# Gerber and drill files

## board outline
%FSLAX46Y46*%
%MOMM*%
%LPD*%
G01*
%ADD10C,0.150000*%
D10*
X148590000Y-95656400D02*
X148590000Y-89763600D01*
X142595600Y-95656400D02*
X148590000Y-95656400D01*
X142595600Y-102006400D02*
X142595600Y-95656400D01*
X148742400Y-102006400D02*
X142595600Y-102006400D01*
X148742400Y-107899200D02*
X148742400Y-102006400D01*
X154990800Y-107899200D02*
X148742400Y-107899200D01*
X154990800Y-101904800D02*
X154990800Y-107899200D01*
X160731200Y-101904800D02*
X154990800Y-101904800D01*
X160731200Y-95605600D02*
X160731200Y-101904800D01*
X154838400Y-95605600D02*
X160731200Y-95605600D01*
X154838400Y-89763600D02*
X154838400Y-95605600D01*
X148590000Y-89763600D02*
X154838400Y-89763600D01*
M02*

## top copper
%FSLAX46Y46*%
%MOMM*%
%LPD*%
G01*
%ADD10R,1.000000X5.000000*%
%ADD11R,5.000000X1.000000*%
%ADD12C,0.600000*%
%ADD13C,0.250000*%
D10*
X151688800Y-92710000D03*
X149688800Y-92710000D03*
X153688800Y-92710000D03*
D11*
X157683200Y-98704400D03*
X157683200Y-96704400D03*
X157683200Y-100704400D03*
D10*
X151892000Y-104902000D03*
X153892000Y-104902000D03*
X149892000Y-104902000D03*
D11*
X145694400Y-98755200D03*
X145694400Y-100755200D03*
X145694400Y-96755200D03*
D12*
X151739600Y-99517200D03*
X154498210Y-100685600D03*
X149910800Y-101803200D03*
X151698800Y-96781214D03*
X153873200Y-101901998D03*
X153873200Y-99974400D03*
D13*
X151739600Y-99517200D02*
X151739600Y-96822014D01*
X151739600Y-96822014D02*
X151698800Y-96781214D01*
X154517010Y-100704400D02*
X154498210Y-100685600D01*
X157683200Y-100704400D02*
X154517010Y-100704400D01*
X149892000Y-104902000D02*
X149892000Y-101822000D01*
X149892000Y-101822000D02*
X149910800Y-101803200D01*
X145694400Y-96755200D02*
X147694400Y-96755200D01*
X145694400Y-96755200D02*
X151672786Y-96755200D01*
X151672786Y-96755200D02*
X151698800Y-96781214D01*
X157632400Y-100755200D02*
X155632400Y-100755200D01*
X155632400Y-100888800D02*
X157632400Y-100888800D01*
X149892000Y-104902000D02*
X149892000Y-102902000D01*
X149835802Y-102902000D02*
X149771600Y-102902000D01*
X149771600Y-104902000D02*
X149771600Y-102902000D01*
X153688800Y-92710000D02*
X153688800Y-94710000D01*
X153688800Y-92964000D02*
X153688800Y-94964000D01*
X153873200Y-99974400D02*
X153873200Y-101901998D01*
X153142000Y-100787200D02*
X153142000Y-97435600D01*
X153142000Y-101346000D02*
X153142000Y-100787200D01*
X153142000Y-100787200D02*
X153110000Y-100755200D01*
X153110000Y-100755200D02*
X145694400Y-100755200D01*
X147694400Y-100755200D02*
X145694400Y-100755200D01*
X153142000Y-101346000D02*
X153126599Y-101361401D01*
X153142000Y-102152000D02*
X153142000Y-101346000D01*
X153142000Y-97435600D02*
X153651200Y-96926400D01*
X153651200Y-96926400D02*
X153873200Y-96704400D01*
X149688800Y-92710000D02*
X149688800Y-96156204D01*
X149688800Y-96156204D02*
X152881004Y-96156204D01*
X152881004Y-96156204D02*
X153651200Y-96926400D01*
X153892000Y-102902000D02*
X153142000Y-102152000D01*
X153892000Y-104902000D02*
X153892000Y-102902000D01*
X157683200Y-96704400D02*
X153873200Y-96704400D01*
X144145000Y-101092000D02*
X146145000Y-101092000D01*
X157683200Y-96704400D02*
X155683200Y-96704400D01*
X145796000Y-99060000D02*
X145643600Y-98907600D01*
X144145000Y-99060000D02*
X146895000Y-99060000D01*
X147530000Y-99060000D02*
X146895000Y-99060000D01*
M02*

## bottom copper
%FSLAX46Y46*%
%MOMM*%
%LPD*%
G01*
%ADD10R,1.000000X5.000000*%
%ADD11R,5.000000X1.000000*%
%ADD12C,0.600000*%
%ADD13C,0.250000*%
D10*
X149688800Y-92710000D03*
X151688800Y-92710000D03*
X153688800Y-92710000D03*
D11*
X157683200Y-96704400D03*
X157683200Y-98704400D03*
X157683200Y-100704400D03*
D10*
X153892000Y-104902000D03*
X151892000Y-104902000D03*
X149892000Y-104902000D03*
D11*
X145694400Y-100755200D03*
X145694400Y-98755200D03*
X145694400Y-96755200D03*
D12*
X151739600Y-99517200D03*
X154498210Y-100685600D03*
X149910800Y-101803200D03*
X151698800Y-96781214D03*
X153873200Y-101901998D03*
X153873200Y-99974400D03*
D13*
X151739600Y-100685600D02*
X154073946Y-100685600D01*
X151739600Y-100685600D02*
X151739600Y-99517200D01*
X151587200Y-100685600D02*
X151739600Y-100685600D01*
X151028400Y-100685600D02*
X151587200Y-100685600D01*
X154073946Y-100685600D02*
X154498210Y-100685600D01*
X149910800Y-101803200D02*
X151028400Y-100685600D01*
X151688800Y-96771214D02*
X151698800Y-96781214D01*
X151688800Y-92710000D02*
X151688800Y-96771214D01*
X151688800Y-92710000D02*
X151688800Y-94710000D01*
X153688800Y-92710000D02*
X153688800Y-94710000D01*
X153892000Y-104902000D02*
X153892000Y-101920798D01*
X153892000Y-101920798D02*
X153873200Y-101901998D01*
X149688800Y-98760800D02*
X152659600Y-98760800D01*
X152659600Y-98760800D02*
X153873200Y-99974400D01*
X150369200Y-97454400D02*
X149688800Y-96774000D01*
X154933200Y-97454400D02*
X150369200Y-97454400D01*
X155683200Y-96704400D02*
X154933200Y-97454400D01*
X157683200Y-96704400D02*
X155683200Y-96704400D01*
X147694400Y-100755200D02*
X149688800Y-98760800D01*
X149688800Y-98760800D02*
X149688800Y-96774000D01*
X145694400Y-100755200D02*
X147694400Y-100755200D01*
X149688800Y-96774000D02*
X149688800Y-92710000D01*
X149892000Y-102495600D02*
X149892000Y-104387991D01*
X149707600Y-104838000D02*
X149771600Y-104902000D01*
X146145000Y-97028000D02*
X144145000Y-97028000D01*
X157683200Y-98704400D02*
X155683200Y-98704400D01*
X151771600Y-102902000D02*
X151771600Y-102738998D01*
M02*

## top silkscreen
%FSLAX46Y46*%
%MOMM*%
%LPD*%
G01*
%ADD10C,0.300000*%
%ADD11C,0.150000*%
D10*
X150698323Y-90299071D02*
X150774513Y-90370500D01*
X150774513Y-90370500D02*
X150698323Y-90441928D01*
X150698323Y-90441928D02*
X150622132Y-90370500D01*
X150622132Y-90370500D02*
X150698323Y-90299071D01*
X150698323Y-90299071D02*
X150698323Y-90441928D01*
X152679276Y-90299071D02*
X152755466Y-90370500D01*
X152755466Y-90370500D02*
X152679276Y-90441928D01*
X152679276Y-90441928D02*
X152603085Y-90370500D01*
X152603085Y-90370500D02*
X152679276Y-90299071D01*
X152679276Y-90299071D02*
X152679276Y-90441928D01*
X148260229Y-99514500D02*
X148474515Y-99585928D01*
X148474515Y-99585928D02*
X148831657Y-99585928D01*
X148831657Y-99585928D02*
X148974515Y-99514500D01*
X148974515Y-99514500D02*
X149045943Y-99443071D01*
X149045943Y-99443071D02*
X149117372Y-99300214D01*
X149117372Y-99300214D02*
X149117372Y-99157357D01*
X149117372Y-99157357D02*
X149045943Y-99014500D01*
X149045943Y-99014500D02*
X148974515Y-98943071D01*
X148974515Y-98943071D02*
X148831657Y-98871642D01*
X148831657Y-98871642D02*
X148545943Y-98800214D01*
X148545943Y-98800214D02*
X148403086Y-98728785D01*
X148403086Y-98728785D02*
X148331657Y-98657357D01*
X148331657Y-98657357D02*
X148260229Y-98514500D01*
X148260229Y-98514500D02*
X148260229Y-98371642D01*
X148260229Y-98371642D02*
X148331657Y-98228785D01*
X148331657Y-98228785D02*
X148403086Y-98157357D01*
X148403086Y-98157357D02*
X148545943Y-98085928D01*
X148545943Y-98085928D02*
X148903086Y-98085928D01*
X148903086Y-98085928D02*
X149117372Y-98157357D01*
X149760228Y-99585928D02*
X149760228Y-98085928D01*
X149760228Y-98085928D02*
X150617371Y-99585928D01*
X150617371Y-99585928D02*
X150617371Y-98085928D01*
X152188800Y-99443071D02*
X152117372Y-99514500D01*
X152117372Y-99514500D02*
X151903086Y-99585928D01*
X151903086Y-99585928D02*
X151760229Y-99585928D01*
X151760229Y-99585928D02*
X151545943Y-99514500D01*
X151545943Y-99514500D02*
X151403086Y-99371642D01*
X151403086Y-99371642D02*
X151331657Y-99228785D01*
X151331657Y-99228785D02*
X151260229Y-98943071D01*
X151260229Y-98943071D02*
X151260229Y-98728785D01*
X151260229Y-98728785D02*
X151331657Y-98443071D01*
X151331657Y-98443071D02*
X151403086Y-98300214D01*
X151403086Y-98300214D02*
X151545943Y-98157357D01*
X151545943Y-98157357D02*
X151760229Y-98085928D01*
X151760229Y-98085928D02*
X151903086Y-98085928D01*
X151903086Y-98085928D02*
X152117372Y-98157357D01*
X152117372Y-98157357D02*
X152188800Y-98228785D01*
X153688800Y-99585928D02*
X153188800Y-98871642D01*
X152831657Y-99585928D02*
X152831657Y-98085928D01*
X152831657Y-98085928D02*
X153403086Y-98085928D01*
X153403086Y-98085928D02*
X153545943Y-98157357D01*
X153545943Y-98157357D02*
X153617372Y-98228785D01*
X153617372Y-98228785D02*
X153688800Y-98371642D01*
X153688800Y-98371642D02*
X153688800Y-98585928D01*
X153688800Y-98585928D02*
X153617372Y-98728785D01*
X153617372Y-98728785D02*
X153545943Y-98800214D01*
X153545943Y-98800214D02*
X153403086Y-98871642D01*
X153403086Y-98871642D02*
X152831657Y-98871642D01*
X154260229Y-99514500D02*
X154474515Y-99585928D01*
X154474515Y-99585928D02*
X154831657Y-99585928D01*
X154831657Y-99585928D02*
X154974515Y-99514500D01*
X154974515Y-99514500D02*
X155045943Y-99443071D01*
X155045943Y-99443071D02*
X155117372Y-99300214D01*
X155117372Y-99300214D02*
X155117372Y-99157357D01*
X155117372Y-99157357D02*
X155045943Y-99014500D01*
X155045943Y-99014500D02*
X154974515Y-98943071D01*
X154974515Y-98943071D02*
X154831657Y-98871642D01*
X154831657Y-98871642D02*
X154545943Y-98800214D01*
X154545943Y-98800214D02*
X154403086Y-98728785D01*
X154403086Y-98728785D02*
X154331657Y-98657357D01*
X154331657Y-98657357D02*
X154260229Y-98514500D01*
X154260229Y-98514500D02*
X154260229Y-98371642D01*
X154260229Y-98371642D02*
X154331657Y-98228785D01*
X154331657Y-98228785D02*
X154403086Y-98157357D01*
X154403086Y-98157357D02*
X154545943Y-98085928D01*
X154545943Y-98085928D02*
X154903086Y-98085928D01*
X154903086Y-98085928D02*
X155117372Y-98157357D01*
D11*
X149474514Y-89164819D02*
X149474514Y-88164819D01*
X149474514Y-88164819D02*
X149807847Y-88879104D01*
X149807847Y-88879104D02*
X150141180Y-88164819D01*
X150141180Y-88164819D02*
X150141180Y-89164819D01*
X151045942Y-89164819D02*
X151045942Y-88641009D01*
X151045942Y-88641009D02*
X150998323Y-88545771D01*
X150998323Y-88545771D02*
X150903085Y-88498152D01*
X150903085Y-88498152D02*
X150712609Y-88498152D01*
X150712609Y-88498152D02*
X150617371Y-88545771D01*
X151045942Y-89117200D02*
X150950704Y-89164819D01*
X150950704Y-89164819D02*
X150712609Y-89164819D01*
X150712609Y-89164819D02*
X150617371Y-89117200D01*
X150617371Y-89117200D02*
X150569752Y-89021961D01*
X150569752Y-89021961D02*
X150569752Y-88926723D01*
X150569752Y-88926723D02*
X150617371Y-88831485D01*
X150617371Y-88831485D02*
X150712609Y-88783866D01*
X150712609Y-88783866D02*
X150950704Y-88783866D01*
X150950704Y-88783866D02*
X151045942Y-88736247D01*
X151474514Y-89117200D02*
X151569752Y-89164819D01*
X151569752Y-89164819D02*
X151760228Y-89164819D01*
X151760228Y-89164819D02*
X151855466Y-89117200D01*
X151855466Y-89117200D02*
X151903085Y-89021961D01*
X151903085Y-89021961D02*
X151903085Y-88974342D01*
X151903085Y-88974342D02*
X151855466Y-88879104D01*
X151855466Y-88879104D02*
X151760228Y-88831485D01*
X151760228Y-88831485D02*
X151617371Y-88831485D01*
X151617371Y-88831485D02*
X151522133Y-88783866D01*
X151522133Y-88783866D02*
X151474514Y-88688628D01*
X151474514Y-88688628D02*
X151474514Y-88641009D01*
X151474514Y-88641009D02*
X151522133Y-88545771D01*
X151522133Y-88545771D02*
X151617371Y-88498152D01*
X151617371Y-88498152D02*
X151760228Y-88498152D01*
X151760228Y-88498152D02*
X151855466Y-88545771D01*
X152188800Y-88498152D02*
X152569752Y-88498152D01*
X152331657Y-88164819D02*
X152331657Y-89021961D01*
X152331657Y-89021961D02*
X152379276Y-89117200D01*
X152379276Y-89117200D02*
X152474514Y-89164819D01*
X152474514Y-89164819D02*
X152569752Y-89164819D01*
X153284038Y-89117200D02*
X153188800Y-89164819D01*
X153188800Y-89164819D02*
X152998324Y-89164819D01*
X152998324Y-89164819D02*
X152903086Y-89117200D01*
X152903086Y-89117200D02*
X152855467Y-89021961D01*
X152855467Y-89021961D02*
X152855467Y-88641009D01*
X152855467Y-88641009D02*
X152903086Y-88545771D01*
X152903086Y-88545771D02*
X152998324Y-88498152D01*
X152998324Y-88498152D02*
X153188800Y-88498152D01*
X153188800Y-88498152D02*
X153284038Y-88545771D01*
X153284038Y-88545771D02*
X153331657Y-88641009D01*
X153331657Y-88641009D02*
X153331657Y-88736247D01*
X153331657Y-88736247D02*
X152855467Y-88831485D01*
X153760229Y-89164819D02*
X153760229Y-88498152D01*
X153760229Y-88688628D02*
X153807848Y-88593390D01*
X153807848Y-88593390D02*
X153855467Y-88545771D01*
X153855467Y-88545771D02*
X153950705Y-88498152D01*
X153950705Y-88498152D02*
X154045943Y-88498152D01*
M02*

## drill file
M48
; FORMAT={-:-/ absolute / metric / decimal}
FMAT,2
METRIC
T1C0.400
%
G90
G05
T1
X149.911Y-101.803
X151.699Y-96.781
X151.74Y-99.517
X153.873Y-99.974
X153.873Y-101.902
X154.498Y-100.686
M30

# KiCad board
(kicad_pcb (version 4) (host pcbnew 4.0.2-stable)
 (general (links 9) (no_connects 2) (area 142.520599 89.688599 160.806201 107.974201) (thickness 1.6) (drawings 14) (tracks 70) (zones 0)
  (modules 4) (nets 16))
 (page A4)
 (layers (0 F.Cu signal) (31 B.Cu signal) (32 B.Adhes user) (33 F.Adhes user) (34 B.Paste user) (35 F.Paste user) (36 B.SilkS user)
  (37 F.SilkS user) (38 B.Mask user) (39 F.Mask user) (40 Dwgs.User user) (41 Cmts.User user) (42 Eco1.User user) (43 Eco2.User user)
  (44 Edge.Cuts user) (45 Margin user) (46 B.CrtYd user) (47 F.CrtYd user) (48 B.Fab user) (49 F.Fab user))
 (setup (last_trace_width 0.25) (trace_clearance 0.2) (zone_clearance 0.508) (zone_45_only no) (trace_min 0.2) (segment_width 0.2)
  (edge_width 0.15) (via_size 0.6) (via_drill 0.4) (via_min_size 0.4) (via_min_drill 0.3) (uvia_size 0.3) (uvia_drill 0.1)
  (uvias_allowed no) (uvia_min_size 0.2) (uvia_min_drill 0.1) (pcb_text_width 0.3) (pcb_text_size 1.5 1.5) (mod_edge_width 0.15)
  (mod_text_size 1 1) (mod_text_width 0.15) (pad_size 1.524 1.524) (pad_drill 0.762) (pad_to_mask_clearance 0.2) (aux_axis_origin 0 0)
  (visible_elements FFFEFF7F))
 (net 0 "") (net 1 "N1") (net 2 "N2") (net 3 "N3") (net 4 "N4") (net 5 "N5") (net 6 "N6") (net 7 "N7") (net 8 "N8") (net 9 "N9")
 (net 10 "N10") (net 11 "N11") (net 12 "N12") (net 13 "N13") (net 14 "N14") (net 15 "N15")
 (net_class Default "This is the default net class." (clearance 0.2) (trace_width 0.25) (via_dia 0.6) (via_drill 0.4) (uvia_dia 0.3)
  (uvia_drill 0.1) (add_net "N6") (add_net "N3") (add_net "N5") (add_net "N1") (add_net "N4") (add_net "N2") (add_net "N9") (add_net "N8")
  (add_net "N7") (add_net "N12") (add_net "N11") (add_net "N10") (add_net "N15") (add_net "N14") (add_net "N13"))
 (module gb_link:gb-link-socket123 (layer F.Cu) (at 151.6888 92.71 180)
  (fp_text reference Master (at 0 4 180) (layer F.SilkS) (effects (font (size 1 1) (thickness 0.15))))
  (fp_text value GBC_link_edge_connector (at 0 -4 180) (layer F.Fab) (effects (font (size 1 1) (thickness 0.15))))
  (pad 4 connect rect (at 0 0 180) (size 1 5) (layers F.Cu F.Mask) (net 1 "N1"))
  (pad 6 connect rect (at 2 0 180) (size 1 5) (layers F.Cu F.Mask) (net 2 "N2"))
  (pad 2 connect rect (at -2 0 180) (size 1 5) (layers F.Cu F.Mask) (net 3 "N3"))
  (pad 5 connect rect (at 2 0 180) (size 1 5) (layers B.Cu B.Mask) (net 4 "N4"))
  (pad 3 connect rect (at 0 0 180) (size 1 5) (layers B.Cu B.Mask) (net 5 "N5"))
  (pad 1 connect rect (at -2 0 180) (size 1 5) (layers B.Cu B.Mask) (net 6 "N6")))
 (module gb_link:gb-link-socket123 (layer F.Cu) (at 157.6832 98.7044 90)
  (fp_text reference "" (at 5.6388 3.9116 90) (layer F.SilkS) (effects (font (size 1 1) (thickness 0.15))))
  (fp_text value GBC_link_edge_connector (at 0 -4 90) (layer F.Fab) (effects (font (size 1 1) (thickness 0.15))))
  (pad 4 connect rect (at 0 0 90) (size 1 5) (layers F.Cu F.Mask) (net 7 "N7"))
  (pad 6 connect rect (at 2 0 90) (size 1 5) (layers F.Cu F.Mask) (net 2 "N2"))
  (pad 2 connect rect (at -2 0 90) (size 1 5) (layers F.Cu F.Mask) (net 5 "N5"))
  (pad 5 connect rect (at 2 0 90) (size 1 5) (layers B.Cu B.Mask) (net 4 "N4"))
  (pad 3 connect rect (at 0 0 90) (size 1 5) (layers B.Cu B.Mask) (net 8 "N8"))
  (pad 1 connect rect (at -2 0 90) (size 1 5) (layers B.Cu B.Mask) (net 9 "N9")))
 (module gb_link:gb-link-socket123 (layer F.Cu) (at 151.892 104.902)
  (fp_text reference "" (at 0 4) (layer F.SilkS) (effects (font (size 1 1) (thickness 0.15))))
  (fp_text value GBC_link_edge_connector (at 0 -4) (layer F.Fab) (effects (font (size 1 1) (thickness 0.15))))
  (pad 4 connect rect (at 0 0) (size 1 5) (layers F.Cu F.Mask) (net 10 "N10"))
  (pad 6 connect rect (at 2 0) (size 1 5) (layers F.Cu F.Mask) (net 2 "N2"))
  (pad 2 connect rect (at -2 0) (size 1 5) (layers F.Cu F.Mask) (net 5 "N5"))
  (pad 5 connect rect (at 2 0) (size 1 5) (layers B.Cu B.Mask) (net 4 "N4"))
  (pad 3 connect rect (at 0 0) (size 1 5) (layers B.Cu B.Mask) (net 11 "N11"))
  (pad 1 connect rect (at -2 0) (size 1 5) (layers B.Cu B.Mask) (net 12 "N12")))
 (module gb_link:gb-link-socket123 (layer F.Cu) (at 145.6944 98.7552 270)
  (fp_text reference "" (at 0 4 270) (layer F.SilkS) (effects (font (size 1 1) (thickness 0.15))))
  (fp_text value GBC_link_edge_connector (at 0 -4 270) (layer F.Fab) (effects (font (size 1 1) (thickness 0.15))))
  (pad 4 connect rect (at 0 0 270) (size 1 5) (layers F.Cu F.Mask) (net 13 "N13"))
  (pad 6 connect rect (at 2 0 270) (size 1 5) (layers F.Cu F.Mask) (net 2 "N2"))
  (pad 2 connect rect (at -2 0 270) (size 1 5) (layers F.Cu F.Mask) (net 5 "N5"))
  (pad 5 connect rect (at 2 0 270) (size 1 5) (layers B.Cu B.Mask) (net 4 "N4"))
  (pad 3 connect rect (at 0 0 270) (size 1 5) (layers B.Cu B.Mask) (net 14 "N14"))
  (pad 1 connect rect (at -2 0 270) (size 1 5) (layers B.Cu B.Mask) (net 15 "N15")))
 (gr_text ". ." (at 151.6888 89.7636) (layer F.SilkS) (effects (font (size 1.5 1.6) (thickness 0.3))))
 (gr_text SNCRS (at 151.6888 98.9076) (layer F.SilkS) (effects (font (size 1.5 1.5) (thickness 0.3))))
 (gr_line (start 148.59 95.6564) (end 148.59 89.7636) (layer Edge.Cuts) (width 0.15))
 (gr_line (start 142.5956 95.6564) (end 148.59 95.6564) (layer Edge.Cuts) (width 0.15))
 (gr_line (start 142.5956 102.0064) (end 142.5956 95.6564) (layer Edge.Cuts) (width 0.15))
 (gr_line (start 148.7424 102.0064) (end 142.5956 102.0064) (layer Edge.Cuts) (width 0.15))
 (gr_line (start 148.7424 107.8992) (end 148.7424 102.0064) (layer Edge.Cuts) (width 0.15))
 (gr_line (start 154.9908 107.8992) (end 148.7424 107.8992) (layer Edge.Cuts) (width 0.15))
 (gr_line (start 154.9908 101.9048) (end 154.9908 107.8992) (layer Edge.Cuts) (width 0.15))
 (gr_line (start 160.7312 101.9048) (end 154.9908 101.9048) (layer Edge.Cuts) (width 0.15))
 (gr_line (start 160.7312 95.6056) (end 160.7312 101.9048) (layer Edge.Cuts) (width 0.15))
 (gr_line (start 154.8384 95.6056) (end 160.7312 95.6056) (layer Edge.Cuts) (width 0.15))
 (gr_line (start 154.8384 89.7636) (end 154.8384 95.6056) (layer Edge.Cuts) (width 0.15))
 (gr_line (start 148.59 89.7636) (end 154.8384 89.7636) (layer Edge.Cuts) (width 0.15))
 (segment (start 151.7396 99.5172) (end 151.7396 96.822014) (width 0.25) (layer F.Cu) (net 5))
 (segment (start 151.7396 96.822014) (end 151.6988 96.781214) (width 0.25) (layer F.Cu) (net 5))
 (segment (start 151.7396 100.6856) (end 154.073946 100.6856) (width 0.25) (layer B.Cu) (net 5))
 (segment (start 151.7396 100.6856) (end 151.7396 99.5172) (width 0.25) (layer B.Cu) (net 5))
 (segment (start 151.5872 100.6856) (end 151.7396 100.6856) (width 0.25) (layer B.Cu) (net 5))
 (via (at 151.7396 99.5172) (size 0.6) (drill 0.4) (layers F.Cu B.Cu) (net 5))
 (segment (start 151.0284 100.6856) (end 151.5872 100.6856) (width 0.25) (layer B.Cu) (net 5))
 (segment (start 154.073946 100.6856) (end 154.49821 100.6856) (width 0.25) (layer B.Cu) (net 5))
 (segment (start 149.9108 101.8032) (end 151.0284 100.6856) (width 0.25) (layer B.Cu) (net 5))
 (segment (start 154.51701 100.7044) (end 154.49821 100.6856) (width 0.25) (layer F.Cu) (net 5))
 (segment (start 157.6832 100.7044) (end 154.51701 100.7044) (width 0.25) (layer F.Cu) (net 5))
 (via (at 154.49821 100.6856) (size 0.6) (drill 0.4) (layers F.Cu B.Cu) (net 5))
 (segment (start 149.892 104.902) (end 149.892 101.822) (width 0.25) (layer F.Cu) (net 5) (status 10))
 (segment (start 149.892 101.822) (end 149.9108 101.8032) (width 0.25) (layer F.Cu) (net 5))
 (via (at 149.9108 101.8032) (size 0.6) (drill 0.4) (layers F.Cu B.Cu) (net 5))
 (segment (start 145.6944 96.7552) (end 147.6944 96.7552) (width 0.25) (layer F.Cu) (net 5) (status 30))
 (segment (start 145.6944 96.7552) (end 151.672786 96.7552) (width 0.25) (layer F.Cu) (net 5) (status 10))
 (segment (start 151.6888 96.771214) (end 151.6988 96.781214) (width 0.25) (layer B.Cu) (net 5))
 (segment (start 151.6888 92.71) (end 151.6888 96.771214) (width 0.25) (layer B.Cu) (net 5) (status 10))
 (segment (start 151.672786 96.7552) (end 151.6988 96.781214) (width 0.25) (layer F.Cu) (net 5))
 (via (at 151.6988 96.781214) (size 0.6) (drill 0.4) (layers F.Cu B.Cu) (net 5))
 (segment (start 151.6888 92.71) (end 151.6888 94.71) (width 0.25) (layer B.Cu) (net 5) (status 30))
 (segment (start 157.6324 100.7552) (end 155.6324 100.7552) (width 0.25) (layer F.Cu) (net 5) (status 30))
 (segment (start 155.6324 100.8888) (end 157.6324 100.8888) (width 0.25) (layer F.Cu) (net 5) (status 30))
 (segment (start 149.892 104.902) (end 149.892 102.902) (width 0.25) (layer F.Cu) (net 5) (status 30))
 (segment (start 149.835802 102.902) (end 149.7716 102.902) (width 0.25) (layer F.Cu) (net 5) (status 30))
 (segment (start 149.7716 104.902) (end 149.7716 102.902) (width 0.25) (layer F.Cu) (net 5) (status 30))
 (segment (start 153.6888 92.71) (end 153.6888 94.71) (width 0.25) (layer B.Cu) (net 6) (status 30))
 (segment (start 153.6888 92.71) (end 153.6888 94.71) (width 0.25) (layer F.Cu) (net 3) (status 30))
 (segment (start 153.6888 92.964) (end 153.6888 94.964) (width 0.25) (layer F.Cu) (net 3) (status 30))
 (segment (start 153.892 104.902) (end 153.892 101.920798) (width 0.25) (layer B.Cu) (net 4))
 (segment (start 153.892 101.920798) (end 153.8732 101.901998) (width 0.25) (layer B.Cu) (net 4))
 (segment (start 153.8732 99.9744) (end 153.8732 101.901998) (width 0.25) (layer F.Cu) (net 4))
 (via (at 153.8732 101.901998) (size 0.6) (drill 0.4) (layers F.Cu B.Cu) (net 4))
 (via (at 153.8732 99.9744) (size 0.6) (drill 0.4) (layers F.Cu B.Cu) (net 4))
 (segment (start 149.6888 98.7608) (end 152.6596 98.7608) (width 0.25) (layer B.Cu) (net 4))
 (segment (start 152.6596 98.7608) (end 153.8732 99.9744) (width 0.25) (layer B.Cu) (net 4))
 (segment (start 150.3692 97.4544) (end 149.6888 96.774) (width 0.25) (layer B.Cu) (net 4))
 (segment (start 154.9332 97.4544) (end 150.3692 97.4544) (width 0.25) (layer B.Cu) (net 4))
 (segment (start 155.6832 96.7044) (end 154.9332 97.4544) (width 0.25) (layer B.Cu) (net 4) (status 10))
 (segment (start 157.6832 96.7044) (end 155.6832 96.7044) (width 0.25) (layer B.Cu) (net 4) (status 30))
 (segment (start 147.6944 100.7552) (end 149.6888 98.7608) (width 0.25) (layer B.Cu) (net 4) (status 10))
 (segment (start 149.6888 98.7608) (end 149.6888 96.774) (width 0.25) (layer B.Cu) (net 4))
 (segment (start 145.6944 100.7552) (end 147.6944 100.7552) (width 0.25) (layer B.Cu) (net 4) (status 30))
 (segment (start 149.6888 96.774) (end 149.6888 92.71) (width 0.25) (layer B.Cu) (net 4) (status 20))
 (segment (start 153.142 100.7872) (end 153.142 97.4356) (width 0.25) (layer F.Cu) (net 2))
 (segment (start 153.142 101.346) (end 153.142 100.7872) (width 0.25) (layer F.Cu) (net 2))
 (segment (start 153.142 100.7872) (end 153.11 100.7552) (width 0.25) (layer F.Cu) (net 2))
 (segment (start 153.11 100.7552) (end 145.6944 100.7552) (width 0.25) (layer F.Cu) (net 2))
 (segment (start 147.6944 100.7552) (end 145.6944 100.7552) (width 0.25) (layer F.Cu) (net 2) (status 30))
 (segment (start 153.142 101.346) (end 153.126599 101.361401) (width 0.25) (layer F.Cu) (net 2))
 (segment (start 153.142 102.152) (end 153.142 101.346) (width 0.25) (layer F.Cu) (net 2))
 (segment (start 153.142 97.4356) (end 153.6512 96.9264) (width 0.25) (layer F.Cu) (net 2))
 (segment (start 153.6512 96.9264) (end 153.8732 96.7044) (width 0.25) (layer F.Cu) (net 2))
 (segment (start 149.6888 92.71) (end 149.6888 96.156204) (width 0.25) (layer F.Cu) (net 2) (status 10))
 (segment (start 149.6888 96.156204) (end 152.881004 96.156204) (width 0.25) (layer F.Cu) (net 2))
 (segment (start 152.881004 96.156204) (end 153.6512 96.9264) (width 0.25) (layer F.Cu) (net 2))
 (segment (start 153.892 102.902) (end 153.142 102.152) (width 0.25) (layer F.Cu) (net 2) (status 10))
 (segment (start 153.892 104.902) (end 153.892 102.902) (width 0.25) (layer F.Cu) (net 2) (status 30))
 (segment (start 157.6832 96.7044) (end 153.8732 96.7044) (width 0.25) (layer F.Cu) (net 2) (status 10))
 (segment (start 144.145 101.092) (end 146.145 101.092) (width 0.25) (layer F.Cu) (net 2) (status 30))
 (segment (start 157.6832 96.7044) (end 155.6832 96.7044) (width 0.25) (layer F.Cu) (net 2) (status 30))
 (segment (start 149.892 102.4956) (end 149.892 104.387991) (width 0.25) (layer B.Cu) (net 12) (status 30))
 (segment (start 149.7076 104.838) (end 149.7716 104.902) (width 0.25) (layer B.Cu) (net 12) (status 30))
 (segment (start 146.145 97.028) (end 144.145 97.028) (width 0.25) (layer B.Cu) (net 15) (status 30))
 (segment (start 145.796 99.06) (end 145.6436 98.9076) (width 0.25) (layer F.Cu) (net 13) (status 30))
 (segment (start 144.145 99.06) (end 146.895 99.06) (width 0.25) (layer F.Cu) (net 13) (status 30))
 (segment (start 147.53 99.06) (end 146.895 99.06) (width 0.25) (layer F.Cu) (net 13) (status 30))
 (segment (start 157.6832 98.7044) (end 155.6832 98.7044) (width 0.25) (layer B.Cu) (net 8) (status 30))
 (segment (start 151.7716 102.902) (end 151.7716 102.738998) (width 0.25) (layer B.Cu) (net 11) (status 30)))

